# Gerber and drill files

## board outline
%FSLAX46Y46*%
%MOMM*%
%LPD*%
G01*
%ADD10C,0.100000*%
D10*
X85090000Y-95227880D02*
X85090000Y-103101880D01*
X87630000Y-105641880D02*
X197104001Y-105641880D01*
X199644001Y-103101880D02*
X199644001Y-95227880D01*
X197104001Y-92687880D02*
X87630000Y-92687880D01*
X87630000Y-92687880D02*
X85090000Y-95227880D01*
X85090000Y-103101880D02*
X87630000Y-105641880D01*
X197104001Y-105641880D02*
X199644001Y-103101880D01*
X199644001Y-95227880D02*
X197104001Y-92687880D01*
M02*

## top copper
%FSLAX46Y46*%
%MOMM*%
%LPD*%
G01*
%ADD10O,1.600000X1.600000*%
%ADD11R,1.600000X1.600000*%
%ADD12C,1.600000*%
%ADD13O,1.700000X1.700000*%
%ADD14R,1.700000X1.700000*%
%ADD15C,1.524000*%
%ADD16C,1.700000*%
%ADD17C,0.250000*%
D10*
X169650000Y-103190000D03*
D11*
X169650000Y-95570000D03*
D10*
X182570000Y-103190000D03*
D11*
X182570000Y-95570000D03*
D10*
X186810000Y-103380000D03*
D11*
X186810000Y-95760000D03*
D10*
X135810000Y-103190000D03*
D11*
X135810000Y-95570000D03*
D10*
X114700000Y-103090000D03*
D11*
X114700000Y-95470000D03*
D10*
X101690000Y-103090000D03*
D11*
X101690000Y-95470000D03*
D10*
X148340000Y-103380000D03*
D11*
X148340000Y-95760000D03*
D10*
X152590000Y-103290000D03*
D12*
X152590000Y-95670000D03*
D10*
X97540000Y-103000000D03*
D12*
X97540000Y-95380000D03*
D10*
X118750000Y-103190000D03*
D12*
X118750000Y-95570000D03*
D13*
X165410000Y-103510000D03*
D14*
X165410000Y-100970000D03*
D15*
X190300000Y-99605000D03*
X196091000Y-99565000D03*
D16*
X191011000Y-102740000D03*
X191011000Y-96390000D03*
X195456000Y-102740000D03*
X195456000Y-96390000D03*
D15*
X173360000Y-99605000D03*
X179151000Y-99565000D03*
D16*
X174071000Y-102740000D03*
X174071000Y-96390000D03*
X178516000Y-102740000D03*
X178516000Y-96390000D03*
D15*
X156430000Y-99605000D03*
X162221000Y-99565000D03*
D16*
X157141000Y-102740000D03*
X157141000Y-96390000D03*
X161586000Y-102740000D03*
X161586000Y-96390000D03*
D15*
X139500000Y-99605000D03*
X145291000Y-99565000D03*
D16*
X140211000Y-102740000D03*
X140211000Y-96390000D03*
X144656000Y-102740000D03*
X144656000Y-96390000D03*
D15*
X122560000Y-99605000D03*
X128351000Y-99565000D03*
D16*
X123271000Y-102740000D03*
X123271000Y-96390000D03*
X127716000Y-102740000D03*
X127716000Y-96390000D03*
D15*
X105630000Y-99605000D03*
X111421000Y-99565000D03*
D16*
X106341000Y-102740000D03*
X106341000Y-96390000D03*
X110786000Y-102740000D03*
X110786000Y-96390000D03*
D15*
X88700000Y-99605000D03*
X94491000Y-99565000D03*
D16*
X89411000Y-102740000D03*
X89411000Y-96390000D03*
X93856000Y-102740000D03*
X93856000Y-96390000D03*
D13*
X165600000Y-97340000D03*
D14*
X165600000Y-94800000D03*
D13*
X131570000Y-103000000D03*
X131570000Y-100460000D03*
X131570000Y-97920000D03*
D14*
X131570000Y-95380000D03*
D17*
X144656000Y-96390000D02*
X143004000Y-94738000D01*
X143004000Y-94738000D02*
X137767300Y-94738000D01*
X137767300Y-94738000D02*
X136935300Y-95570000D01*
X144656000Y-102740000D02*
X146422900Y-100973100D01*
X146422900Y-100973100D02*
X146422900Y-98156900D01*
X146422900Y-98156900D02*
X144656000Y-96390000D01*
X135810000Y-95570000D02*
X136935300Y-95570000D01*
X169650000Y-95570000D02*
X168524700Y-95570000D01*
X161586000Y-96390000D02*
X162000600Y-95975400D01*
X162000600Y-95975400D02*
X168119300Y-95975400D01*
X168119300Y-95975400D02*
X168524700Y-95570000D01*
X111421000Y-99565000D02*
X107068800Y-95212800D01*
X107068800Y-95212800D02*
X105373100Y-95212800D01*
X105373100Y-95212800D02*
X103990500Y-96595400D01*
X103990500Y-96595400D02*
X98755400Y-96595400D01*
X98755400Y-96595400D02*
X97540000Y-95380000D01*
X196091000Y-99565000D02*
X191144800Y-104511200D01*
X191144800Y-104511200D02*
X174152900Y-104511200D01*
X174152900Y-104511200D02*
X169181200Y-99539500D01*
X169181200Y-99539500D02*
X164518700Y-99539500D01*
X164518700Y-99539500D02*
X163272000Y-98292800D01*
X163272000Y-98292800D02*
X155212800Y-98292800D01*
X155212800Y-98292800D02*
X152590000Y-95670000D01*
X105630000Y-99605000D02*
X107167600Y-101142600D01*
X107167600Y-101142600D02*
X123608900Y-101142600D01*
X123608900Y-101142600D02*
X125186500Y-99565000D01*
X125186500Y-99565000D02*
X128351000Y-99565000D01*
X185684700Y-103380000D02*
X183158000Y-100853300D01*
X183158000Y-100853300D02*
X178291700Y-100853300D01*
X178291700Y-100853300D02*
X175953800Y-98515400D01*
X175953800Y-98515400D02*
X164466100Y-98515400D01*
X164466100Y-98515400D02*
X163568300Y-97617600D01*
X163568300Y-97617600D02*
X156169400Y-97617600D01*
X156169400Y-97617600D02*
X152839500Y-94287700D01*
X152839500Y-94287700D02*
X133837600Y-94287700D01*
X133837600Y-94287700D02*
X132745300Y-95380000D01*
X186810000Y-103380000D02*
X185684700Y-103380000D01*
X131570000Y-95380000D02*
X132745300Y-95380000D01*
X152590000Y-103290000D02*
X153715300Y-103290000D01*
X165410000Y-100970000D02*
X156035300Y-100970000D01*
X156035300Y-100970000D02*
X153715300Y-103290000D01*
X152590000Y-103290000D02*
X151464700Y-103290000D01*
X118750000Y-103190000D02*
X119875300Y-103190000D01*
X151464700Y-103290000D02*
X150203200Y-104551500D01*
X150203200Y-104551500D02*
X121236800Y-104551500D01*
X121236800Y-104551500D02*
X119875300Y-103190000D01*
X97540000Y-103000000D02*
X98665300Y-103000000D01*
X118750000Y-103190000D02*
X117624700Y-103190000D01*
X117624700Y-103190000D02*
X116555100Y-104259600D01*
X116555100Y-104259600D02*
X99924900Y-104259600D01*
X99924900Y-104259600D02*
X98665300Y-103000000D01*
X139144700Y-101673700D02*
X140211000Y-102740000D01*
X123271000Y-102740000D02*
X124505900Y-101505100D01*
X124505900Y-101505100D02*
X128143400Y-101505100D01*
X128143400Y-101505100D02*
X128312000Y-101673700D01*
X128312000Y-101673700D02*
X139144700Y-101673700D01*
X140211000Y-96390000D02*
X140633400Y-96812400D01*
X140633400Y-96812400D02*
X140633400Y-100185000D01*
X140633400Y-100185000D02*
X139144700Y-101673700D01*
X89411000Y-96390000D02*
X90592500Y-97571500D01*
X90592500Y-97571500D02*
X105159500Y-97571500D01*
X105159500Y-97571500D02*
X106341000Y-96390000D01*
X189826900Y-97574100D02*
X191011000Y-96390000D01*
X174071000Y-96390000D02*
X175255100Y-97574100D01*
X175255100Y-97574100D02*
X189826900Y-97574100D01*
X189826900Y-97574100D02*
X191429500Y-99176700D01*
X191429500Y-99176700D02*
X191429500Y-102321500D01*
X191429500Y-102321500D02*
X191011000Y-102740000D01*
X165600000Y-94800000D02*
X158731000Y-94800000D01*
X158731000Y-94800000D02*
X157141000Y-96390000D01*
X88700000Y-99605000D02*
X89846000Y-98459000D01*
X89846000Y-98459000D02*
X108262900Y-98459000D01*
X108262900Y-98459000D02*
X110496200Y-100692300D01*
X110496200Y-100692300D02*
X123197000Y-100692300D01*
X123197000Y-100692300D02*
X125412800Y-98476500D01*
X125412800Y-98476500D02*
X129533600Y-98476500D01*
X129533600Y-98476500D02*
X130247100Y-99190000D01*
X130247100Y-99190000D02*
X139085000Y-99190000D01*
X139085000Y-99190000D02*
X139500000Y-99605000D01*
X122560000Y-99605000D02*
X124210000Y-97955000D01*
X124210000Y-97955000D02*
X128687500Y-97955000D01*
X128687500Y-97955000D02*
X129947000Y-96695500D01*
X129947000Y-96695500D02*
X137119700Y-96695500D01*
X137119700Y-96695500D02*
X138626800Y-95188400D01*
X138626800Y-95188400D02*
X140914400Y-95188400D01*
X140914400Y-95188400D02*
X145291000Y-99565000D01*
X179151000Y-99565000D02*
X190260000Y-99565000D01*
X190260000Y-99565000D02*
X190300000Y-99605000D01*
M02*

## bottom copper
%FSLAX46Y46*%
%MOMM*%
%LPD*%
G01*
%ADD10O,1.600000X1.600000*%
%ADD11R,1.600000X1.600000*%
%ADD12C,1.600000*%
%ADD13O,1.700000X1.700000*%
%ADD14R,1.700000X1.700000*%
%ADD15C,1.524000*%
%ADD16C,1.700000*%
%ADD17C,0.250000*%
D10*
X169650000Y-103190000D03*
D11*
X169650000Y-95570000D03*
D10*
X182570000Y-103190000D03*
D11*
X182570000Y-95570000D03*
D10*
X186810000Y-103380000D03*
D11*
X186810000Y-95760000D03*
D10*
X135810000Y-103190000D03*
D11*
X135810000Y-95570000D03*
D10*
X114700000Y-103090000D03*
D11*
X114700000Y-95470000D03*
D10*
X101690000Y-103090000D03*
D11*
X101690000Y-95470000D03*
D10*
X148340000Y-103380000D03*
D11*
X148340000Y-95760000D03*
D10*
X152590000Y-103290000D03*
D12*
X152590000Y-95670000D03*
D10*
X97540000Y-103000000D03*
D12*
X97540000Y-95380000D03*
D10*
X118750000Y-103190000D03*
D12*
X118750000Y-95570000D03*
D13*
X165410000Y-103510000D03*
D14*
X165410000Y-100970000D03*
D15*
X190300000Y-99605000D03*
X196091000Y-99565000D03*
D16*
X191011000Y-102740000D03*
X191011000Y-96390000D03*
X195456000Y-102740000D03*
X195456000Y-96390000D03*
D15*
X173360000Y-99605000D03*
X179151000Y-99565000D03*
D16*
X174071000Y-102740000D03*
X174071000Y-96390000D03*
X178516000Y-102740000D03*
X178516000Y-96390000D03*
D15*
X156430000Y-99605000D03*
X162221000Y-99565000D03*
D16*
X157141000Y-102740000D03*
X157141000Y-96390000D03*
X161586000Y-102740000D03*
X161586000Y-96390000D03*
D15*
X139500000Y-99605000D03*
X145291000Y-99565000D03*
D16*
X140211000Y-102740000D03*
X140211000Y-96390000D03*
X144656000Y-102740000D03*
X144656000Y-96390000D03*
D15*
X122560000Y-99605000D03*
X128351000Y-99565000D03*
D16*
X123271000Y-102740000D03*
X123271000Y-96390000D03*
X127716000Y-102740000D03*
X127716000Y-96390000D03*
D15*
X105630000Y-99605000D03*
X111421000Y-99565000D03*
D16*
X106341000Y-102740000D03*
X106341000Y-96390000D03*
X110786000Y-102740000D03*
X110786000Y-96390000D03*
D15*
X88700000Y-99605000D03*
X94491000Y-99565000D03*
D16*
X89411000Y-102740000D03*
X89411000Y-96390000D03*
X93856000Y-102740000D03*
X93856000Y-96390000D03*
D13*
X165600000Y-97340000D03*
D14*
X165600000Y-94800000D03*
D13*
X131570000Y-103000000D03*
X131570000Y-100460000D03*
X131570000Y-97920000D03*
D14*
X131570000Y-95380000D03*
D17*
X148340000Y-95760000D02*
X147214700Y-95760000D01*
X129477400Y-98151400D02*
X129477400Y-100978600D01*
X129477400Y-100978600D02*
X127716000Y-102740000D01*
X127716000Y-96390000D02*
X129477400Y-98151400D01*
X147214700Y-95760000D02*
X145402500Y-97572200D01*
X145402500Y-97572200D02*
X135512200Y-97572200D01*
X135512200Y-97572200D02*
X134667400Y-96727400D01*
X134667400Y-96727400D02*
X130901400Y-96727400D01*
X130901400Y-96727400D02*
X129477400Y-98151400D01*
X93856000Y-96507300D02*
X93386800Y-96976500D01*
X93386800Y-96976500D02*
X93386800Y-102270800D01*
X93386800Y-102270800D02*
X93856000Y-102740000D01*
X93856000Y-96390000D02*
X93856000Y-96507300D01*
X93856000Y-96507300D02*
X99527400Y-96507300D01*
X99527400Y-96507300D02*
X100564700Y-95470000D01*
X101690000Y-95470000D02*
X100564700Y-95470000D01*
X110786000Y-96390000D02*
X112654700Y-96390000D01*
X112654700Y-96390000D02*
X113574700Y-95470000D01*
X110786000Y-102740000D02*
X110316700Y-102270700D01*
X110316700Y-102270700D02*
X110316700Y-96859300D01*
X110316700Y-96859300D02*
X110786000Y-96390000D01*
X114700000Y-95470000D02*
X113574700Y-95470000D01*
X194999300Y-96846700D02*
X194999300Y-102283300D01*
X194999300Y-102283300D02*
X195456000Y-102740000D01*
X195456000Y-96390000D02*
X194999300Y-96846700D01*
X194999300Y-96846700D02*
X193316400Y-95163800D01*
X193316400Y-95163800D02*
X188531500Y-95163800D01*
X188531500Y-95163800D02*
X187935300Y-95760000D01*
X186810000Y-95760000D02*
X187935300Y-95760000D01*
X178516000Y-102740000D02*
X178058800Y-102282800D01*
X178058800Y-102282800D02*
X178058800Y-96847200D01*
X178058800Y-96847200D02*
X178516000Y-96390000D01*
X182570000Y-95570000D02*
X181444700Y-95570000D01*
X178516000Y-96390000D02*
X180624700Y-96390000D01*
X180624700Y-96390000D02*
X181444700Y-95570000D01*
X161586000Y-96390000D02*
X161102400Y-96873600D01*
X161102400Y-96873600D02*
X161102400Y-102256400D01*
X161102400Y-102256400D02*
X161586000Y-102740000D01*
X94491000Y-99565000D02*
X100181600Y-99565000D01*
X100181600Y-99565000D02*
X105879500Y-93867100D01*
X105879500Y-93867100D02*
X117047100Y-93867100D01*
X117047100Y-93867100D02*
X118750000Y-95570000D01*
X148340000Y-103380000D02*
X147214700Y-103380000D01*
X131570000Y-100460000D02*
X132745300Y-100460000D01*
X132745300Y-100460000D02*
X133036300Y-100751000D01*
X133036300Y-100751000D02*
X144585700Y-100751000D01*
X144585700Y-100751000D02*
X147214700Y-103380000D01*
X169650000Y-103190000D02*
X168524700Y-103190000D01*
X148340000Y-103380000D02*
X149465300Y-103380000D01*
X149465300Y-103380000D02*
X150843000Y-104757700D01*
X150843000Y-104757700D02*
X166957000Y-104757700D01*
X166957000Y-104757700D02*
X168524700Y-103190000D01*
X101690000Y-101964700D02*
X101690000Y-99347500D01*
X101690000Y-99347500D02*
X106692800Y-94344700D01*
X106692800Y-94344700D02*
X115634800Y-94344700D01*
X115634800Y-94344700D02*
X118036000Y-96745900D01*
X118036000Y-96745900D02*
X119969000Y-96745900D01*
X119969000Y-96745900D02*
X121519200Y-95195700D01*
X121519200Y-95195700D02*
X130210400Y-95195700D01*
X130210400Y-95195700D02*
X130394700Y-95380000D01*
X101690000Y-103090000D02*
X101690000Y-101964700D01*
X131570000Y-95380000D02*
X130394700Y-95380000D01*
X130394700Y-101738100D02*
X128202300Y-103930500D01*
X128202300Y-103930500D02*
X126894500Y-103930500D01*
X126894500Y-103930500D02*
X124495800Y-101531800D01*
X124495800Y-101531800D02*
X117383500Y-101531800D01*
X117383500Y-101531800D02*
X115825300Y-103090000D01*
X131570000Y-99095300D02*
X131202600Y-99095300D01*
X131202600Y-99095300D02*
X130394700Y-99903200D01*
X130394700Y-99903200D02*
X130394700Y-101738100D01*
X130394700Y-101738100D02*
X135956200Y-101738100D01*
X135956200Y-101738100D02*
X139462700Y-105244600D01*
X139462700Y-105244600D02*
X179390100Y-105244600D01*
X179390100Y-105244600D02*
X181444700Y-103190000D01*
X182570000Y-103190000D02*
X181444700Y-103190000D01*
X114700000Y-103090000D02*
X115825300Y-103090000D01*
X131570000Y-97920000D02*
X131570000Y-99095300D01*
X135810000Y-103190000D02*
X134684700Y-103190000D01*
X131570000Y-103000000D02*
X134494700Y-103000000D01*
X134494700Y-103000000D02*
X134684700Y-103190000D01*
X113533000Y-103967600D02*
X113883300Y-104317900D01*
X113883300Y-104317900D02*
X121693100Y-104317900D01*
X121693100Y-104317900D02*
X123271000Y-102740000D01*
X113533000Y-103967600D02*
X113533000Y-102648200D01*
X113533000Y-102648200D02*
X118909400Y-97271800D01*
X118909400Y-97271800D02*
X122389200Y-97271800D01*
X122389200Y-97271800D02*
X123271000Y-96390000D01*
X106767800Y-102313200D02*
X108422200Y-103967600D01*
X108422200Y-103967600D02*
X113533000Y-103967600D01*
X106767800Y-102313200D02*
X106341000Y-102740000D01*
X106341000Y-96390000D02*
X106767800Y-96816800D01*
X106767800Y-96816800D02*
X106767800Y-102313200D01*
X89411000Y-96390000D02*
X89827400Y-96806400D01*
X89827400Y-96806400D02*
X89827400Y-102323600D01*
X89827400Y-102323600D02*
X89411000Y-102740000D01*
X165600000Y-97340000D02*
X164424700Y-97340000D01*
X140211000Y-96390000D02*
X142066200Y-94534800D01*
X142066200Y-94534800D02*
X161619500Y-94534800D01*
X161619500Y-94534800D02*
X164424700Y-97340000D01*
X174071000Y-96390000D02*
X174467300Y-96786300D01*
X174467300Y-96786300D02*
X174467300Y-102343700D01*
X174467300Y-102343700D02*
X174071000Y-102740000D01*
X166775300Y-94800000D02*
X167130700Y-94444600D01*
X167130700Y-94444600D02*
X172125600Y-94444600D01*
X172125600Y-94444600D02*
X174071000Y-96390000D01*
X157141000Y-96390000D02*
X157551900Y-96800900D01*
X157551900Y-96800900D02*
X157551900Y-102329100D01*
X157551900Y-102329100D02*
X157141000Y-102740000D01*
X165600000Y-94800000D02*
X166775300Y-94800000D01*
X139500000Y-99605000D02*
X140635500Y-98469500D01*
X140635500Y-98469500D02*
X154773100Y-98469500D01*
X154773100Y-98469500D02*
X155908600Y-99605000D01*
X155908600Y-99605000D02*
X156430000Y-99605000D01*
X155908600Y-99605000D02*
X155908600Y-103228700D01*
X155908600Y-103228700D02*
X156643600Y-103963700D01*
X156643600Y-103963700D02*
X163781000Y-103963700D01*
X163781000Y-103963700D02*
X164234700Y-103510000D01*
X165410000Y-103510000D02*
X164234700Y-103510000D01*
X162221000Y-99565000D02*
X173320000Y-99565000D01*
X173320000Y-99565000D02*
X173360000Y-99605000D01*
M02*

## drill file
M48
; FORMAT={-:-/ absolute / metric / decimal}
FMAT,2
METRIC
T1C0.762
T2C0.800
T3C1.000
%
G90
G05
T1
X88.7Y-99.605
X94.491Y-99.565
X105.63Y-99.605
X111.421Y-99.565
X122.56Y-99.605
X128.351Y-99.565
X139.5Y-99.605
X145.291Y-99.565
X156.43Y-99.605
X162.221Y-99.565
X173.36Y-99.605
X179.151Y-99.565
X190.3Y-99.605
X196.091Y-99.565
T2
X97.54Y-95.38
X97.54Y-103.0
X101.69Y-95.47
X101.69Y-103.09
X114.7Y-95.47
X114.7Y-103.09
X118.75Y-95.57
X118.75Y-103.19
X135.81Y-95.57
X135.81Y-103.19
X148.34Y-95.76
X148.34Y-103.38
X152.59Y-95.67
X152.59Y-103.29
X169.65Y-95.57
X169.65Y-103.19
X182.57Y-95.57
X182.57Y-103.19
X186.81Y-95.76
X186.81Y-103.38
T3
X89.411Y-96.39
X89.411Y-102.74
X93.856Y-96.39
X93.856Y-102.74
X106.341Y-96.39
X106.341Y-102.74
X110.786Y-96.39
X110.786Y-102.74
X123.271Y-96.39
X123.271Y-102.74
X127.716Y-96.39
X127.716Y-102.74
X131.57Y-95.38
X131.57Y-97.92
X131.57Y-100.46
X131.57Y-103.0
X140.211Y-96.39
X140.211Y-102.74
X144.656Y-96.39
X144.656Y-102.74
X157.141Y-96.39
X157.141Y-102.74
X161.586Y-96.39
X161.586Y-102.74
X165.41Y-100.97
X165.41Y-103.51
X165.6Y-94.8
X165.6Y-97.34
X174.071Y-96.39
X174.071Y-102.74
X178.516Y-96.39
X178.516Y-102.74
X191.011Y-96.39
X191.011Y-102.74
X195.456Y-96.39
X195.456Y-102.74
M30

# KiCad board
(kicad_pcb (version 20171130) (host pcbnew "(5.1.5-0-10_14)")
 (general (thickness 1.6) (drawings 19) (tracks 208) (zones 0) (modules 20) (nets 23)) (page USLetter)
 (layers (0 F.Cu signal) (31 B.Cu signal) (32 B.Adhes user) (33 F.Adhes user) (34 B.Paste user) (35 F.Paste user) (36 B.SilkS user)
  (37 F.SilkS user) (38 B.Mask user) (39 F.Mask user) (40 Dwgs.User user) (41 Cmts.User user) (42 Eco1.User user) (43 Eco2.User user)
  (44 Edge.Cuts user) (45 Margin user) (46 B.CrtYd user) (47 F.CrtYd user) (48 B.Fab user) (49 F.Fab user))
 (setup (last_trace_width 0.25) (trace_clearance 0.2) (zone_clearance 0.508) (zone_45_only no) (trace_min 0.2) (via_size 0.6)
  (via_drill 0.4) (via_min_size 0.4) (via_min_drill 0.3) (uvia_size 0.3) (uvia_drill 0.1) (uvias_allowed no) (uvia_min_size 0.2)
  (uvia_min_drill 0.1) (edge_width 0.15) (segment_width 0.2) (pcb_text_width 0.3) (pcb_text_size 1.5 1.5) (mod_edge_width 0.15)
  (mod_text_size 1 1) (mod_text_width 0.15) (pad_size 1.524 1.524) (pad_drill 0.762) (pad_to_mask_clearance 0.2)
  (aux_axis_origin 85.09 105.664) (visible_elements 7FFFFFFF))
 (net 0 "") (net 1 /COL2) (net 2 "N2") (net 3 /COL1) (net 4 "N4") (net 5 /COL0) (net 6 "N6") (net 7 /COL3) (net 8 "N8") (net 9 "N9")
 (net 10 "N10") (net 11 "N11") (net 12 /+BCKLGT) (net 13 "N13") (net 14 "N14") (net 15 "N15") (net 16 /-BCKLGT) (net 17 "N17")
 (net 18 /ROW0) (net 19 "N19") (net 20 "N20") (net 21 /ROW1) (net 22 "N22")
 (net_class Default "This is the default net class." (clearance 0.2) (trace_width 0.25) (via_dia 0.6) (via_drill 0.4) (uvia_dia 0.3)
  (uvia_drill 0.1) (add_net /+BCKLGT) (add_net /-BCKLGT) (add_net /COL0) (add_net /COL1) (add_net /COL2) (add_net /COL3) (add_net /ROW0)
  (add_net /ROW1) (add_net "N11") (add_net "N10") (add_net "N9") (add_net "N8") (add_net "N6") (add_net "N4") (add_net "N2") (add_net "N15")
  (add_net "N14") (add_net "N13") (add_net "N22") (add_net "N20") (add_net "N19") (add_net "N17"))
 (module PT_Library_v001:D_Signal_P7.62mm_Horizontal (layer F.Cu) (at 169.65 95.57 270)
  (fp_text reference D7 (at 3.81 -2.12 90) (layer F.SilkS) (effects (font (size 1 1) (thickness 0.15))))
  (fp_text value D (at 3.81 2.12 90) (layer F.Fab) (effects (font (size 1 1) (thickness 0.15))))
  (pad 2 thru_hole oval (at 7.62 0 270) (size 1.6 1.6) (drill 0.8) (layers *.Cu *.Mask) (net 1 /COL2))
  (pad 1 thru_hole rect (at 0 0 270) (size 1.6 1.6) (drill 0.8) (layers *.Cu *.Mask) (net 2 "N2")))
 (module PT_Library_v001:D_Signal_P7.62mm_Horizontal (layer F.Cu) (at 182.57 95.57 270)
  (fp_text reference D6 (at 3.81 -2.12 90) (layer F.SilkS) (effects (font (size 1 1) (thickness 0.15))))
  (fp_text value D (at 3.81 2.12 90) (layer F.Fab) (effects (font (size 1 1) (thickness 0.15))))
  (pad 2 thru_hole oval (at 7.62 0 270) (size 1.6 1.6) (drill 0.8) (layers *.Cu *.Mask) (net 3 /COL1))
  (pad 1 thru_hole rect (at 0 0 270) (size 1.6 1.6) (drill 0.8) (layers *.Cu *.Mask) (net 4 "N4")))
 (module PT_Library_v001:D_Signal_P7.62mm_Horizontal (layer F.Cu) (at 186.81 95.76 270)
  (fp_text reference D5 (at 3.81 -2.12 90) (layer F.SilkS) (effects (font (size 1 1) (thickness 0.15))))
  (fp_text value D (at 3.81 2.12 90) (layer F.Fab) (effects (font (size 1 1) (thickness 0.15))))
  (pad 2 thru_hole oval (at 7.62 0 270) (size 1.6 1.6) (drill 0.8) (layers *.Cu *.Mask) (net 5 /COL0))
  (pad 1 thru_hole rect (at 0 0 270) (size 1.6 1.6) (drill 0.8) (layers *.Cu *.Mask) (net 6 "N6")))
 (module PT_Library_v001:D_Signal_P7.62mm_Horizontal (layer F.Cu) (at 135.81 95.57 270)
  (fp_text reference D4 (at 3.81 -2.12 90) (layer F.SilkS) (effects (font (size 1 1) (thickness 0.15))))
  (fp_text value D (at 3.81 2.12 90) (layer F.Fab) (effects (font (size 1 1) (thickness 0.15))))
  (pad 2 thru_hole oval (at 7.62 0 270) (size 1.6 1.6) (drill 0.8) (layers *.Cu *.Mask) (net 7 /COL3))
  (pad 1 thru_hole rect (at 0 0 270) (size 1.6 1.6) (drill 0.8) (layers *.Cu *.Mask) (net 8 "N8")))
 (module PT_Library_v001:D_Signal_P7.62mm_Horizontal (layer F.Cu) (at 114.7 95.47 270)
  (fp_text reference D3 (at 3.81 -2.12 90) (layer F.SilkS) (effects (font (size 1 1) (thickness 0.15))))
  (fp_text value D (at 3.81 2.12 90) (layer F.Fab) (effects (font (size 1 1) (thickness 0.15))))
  (pad 2 thru_hole oval (at 7.62 0 270) (size 1.6 1.6) (drill 0.8) (layers *.Cu *.Mask) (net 3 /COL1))
  (pad 1 thru_hole rect (at 0 0 270) (size 1.6 1.6) (drill 0.8) (layers *.Cu *.Mask) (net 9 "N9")))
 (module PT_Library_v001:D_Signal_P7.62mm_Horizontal (layer F.Cu) (at 101.69 95.47 270)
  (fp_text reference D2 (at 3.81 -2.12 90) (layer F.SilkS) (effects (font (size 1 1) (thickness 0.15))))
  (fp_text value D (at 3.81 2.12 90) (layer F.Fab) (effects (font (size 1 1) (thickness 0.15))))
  (pad 2 thru_hole oval (at 7.62 0 270) (size 1.6 1.6) (drill 0.8) (layers *.Cu *.Mask) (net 5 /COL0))
  (pad 1 thru_hole rect (at 0 0 270) (size 1.6 1.6) (drill 0.8) (layers *.Cu *.Mask) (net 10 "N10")))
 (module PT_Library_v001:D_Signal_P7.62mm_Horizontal (layer F.Cu) (at 148.34 95.76 270)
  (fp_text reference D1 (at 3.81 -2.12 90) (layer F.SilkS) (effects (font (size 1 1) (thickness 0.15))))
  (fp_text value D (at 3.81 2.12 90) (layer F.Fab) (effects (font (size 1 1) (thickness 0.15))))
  (pad 2 thru_hole oval (at 7.62 0 270) (size 1.6 1.6) (drill 0.8) (layers *.Cu *.Mask) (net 1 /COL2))
  (pad 1 thru_hole rect (at 0 0 270) (size 1.6 1.6) (drill 0.8) (layers *.Cu *.Mask) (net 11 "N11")))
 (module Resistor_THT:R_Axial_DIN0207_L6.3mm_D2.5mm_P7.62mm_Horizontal (layer F.Cu) (at 152.59 95.67 270)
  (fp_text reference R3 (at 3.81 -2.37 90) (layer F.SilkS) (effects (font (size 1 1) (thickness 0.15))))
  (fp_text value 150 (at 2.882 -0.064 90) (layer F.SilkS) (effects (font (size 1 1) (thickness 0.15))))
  (pad 2 thru_hole oval (at 7.62 0 270) (size 1.6 1.6) (drill 0.8) (layers *.Cu *.Mask) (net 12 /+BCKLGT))
  (pad 1 thru_hole circle (at 0 0 270) (size 1.6 1.6) (drill 0.8) (layers *.Cu *.Mask) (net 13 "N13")))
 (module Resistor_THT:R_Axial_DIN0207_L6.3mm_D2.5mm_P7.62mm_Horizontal (layer F.Cu) (at 97.54 95.38 270)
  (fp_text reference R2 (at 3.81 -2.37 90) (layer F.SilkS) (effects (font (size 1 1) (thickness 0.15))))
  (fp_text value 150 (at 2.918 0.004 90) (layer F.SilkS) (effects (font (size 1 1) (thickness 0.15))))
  (pad 2 thru_hole oval (at 7.62 0 270) (size 1.6 1.6) (drill 0.8) (layers *.Cu *.Mask) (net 12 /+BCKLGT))
  (pad 1 thru_hole circle (at 0 0 270) (size 1.6 1.6) (drill 0.8) (layers *.Cu *.Mask) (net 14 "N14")))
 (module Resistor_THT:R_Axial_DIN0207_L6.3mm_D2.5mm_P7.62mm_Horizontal (layer F.Cu) (at 118.75 95.57 270)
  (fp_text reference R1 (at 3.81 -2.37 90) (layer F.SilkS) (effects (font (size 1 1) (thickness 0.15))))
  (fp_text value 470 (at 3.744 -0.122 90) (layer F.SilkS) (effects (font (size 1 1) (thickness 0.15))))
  (pad 2 thru_hole oval (at 7.62 0 270) (size 1.6 1.6) (drill 0.8) (layers *.Cu *.Mask) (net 12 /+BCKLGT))
  (pad 1 thru_hole circle (at 0 0 270) (size 1.6 1.6) (drill 0.8) (layers *.Cu *.Mask) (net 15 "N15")))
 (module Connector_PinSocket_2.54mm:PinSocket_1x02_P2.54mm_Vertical (layer B.Cu) (at 165.41 100.97 180)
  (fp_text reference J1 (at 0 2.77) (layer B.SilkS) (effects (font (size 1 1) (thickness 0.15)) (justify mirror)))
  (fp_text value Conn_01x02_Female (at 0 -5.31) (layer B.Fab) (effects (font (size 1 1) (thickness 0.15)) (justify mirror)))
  (pad 2 thru_hole oval (at 0 -2.54 180) (size 1.7 1.7) (drill 1) (layers *.Cu *.Mask) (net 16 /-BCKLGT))
  (pad 1 thru_hole rect (at 0 0 180) (size 1.7 1.7) (drill 1) (layers *.Cu *.Mask) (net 12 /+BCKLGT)))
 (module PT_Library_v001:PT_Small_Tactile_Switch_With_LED (layer F.Cu) (at 193.17 99.565 270)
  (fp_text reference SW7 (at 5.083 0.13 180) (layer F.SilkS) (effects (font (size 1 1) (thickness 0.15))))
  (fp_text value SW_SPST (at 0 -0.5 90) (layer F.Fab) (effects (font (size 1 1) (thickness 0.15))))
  (pad 6 thru_hole circle (at 0.04 2.87 270) (size 1.524 1.524) (drill 0.762) (layers *.Cu *.Mask) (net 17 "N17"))
  (pad 5 thru_hole circle (at 0 -2.921 270) (size 1.524 1.524) (drill 0.762) (layers *.Cu *.Mask) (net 13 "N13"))
  (pad 4 thru_hole circle (at 3.175 2.159 270) (size 1.7 1.7) (drill 1) (layers *.Cu *.Mask) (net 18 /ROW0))
  (pad 3 thru_hole circle (at -3.175 2.159 270) (size 1.7 1.7) (drill 1) (layers *.Cu *.Mask) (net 18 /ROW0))
  (pad 2 thru_hole circle (at 3.175 -2.286 270) (size 1.7 1.7) (drill 1) (layers *.Cu *.Mask) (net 6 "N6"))
  (pad 1 thru_hole circle (at -3.175 -2.286 270) (size 1.7 1.7) (drill 1) (layers *.Cu *.Mask) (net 6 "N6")))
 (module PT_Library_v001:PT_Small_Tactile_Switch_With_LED (layer F.Cu) (at 176.23 99.565 270)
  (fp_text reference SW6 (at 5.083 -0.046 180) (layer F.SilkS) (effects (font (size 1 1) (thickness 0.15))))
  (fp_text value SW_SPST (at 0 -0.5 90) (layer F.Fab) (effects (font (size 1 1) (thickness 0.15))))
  (pad 6 thru_hole circle (at 0.04 2.87 270) (size 1.524 1.524) (drill 0.762) (layers *.Cu *.Mask) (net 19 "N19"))
  (pad 5 thru_hole circle (at 0 -2.921 270) (size 1.524 1.524) (drill 0.762) (layers *.Cu *.Mask) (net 17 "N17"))
  (pad 4 thru_hole circle (at 3.175 2.159 270) (size 1.7 1.7) (drill 1) (layers *.Cu *.Mask) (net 18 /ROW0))
  (pad 3 thru_hole circle (at -3.175 2.159 270) (size 1.7 1.7) (drill 1) (layers *.Cu *.Mask) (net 18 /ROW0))
  (pad 2 thru_hole circle (at 3.175 -2.286 270) (size 1.7 1.7) (drill 1) (layers *.Cu *.Mask) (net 4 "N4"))
  (pad 1 thru_hole circle (at -3.175 -2.286 270) (size 1.7 1.7) (drill 1) (layers *.Cu *.Mask) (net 4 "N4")))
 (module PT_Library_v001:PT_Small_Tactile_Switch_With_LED (layer F.Cu) (at 159.3 99.565 270)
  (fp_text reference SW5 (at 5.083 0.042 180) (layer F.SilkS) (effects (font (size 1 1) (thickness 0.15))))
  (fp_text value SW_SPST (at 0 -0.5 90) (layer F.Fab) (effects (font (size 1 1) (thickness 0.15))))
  (pad 6 thru_hole circle (at 0.04 2.87 270) (size 1.524 1.524) (drill 0.762) (layers *.Cu *.Mask) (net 16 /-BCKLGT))
  (pad 5 thru_hole circle (at 0 -2.921 270) (size 1.524 1.524) (drill 0.762) (layers *.Cu *.Mask) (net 19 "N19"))
  (pad 4 thru_hole circle (at 3.175 2.159 270) (size 1.7 1.7) (drill 1) (layers *.Cu *.Mask) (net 18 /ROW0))
  (pad 3 thru_hole circle (at -3.175 2.159 270) (size 1.7 1.7) (drill 1) (layers *.Cu *.Mask) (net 18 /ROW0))
  (pad 2 thru_hole circle (at 3.175 -2.286 270) (size 1.7 1.7) (drill 1) (layers *.Cu *.Mask) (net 2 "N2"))
  (pad 1 thru_hole circle (at -3.175 -2.286 270) (size 1.7 1.7) (drill 1) (layers *.Cu *.Mask) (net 2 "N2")))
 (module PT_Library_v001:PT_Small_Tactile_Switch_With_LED (layer F.Cu) (at 142.37 99.565 270)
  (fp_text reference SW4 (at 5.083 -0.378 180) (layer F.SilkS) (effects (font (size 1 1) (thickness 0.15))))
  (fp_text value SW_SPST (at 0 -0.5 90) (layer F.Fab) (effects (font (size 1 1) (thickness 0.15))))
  (pad 6 thru_hole circle (at 0.04 2.87 270) (size 1.524 1.524) (drill 0.762) (layers *.Cu *.Mask) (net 16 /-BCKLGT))
  (pad 5 thru_hole circle (at 0 -2.921 270) (size 1.524 1.524) (drill 0.762) (layers *.Cu *.Mask) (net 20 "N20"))
  (pad 4 thru_hole circle (at 3.175 2.159 270) (size 1.7 1.7) (drill 1) (layers *.Cu *.Mask) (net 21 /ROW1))
  (pad 3 thru_hole circle (at -3.175 2.159 270) (size 1.7 1.7) (drill 1) (layers *.Cu *.Mask) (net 21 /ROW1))
  (pad 2 thru_hole circle (at 3.175 -2.286 270) (size 1.7 1.7) (drill 1) (layers *.Cu *.Mask) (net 8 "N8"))
  (pad 1 thru_hole circle (at -3.175 -2.286 270) (size 1.7 1.7) (drill 1) (layers *.Cu *.Mask) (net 8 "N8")))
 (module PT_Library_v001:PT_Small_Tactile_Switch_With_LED (layer F.Cu) (at 125.43 99.565 270)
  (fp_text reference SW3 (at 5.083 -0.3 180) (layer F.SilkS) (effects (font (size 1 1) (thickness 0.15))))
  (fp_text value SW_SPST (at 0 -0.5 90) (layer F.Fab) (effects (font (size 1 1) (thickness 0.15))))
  (pad 6 thru_hole circle (at 0.04 2.87 270) (size 1.524 1.524) (drill 0.762) (layers *.Cu *.Mask) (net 20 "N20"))
  (pad 5 thru_hole circle (at 0 -2.921 270) (size 1.524 1.524) (drill 0.762) (layers *.Cu *.Mask) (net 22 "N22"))
  (pad 4 thru_hole circle (at 3.175 2.159 270) (size 1.7 1.7) (drill 1) (layers *.Cu *.Mask) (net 21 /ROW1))
  (pad 3 thru_hole circle (at -3.175 2.159 270) (size 1.7 1.7) (drill 1) (layers *.Cu *.Mask) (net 21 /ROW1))
  (pad 2 thru_hole circle (at 3.175 -2.286 270) (size 1.7 1.7) (drill 1) (layers *.Cu *.Mask) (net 11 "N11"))
  (pad 1 thru_hole circle (at -3.175 -2.286 270) (size 1.7 1.7) (drill 1) (layers *.Cu *.Mask) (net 11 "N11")))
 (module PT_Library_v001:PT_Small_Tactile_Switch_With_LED (layer F.Cu) (at 108.5 99.565 270)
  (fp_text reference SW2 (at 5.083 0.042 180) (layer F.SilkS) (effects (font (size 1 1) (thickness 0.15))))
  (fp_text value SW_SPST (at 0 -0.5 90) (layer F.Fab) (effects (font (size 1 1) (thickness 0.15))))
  (pad 6 thru_hole circle (at 0.04 2.87 270) (size 1.524 1.524) (drill 0.762) (layers *.Cu *.Mask) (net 22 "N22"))
  (pad 5 thru_hole circle (at 0 -2.921 270) (size 1.524 1.524) (drill 0.762) (layers *.Cu *.Mask) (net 14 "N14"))
  (pad 4 thru_hole circle (at 3.175 2.159 270) (size 1.7 1.7) (drill 1) (layers *.Cu *.Mask) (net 21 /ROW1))
  (pad 3 thru_hole circle (at -3.175 2.159 270) (size 1.7 1.7) (drill 1) (layers *.Cu *.Mask) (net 21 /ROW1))
  (pad 2 thru_hole circle (at 3.175 -2.286 270) (size 1.7 1.7) (drill 1) (layers *.Cu *.Mask) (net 9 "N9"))
  (pad 1 thru_hole circle (at -3.175 -2.286 270) (size 1.7 1.7) (drill 1) (layers *.Cu *.Mask) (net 9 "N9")))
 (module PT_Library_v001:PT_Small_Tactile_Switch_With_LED (layer F.Cu) (at 91.57 99.565 270)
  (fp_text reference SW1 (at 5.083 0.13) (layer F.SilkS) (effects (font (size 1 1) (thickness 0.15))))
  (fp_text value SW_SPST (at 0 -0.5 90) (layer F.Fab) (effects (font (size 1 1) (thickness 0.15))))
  (pad 6 thru_hole circle (at 0.04 2.87 270) (size 1.524 1.524) (drill 0.762) (layers *.Cu *.Mask) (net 16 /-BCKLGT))
  (pad 5 thru_hole circle (at 0 -2.921 270) (size 1.524 1.524) (drill 0.762) (layers *.Cu *.Mask) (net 15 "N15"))
  (pad 4 thru_hole circle (at 3.175 2.159 270) (size 1.7 1.7) (drill 1) (layers *.Cu *.Mask) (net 21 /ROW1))
  (pad 3 thru_hole circle (at -3.175 2.159 270) (size 1.7 1.7) (drill 1) (layers *.Cu *.Mask) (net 21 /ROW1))
  (pad 2 thru_hole circle (at 3.175 -2.286 270) (size 1.7 1.7) (drill 1) (layers *.Cu *.Mask) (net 10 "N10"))
  (pad 1 thru_hole circle (at -3.175 -2.286 270) (size 1.7 1.7) (drill 1) (layers *.Cu *.Mask) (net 10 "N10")))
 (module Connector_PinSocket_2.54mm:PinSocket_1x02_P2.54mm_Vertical (layer B.Cu) (at 165.6 94.8 180)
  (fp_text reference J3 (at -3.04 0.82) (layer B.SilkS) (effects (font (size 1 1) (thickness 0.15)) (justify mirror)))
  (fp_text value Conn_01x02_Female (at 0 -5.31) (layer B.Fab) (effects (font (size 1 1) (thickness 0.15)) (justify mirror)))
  (pad 2 thru_hole oval (at 0 -2.54 180) (size 1.7 1.7) (drill 1) (layers *.Cu *.Mask) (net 21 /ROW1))
  (pad 1 thru_hole rect (at 0 0 180) (size 1.7 1.7) (drill 1) (layers *.Cu *.Mask) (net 18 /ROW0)))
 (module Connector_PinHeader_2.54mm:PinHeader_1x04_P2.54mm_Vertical (layer B.Cu) (at 131.57 95.38 180)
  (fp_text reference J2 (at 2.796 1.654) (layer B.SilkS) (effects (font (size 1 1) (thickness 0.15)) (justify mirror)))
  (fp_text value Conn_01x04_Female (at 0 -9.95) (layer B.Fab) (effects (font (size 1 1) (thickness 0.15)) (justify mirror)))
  (pad 4 thru_hole oval (at 0 -7.62 180) (size 1.7 1.7) (drill 1) (layers *.Cu *.Mask) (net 7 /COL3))
  (pad 3 thru_hole oval (at 0 -5.08 180) (size 1.7 1.7) (drill 1) (layers *.Cu *.Mask) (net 1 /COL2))
  (pad 2 thru_hole oval (at 0 -2.54 180) (size 1.7 1.7) (drill 1) (layers *.Cu *.Mask) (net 3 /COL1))
  (pad 1 thru_hole rect (at 0 0 180) (size 1.7 1.7) (drill 1) (layers *.Cu *.Mask) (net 5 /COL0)))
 (gr_line (start 85.09 95.22788) (end 85.09 103.10188) (layer Edge.Cuts) (width 0.1))
 (gr_line (start 87.63 105.64188) (end 197.104001 105.64188) (layer Edge.Cuts) (width 0.1))
 (gr_line (start 199.644001 103.10188) (end 199.644001 95.22788) (layer Edge.Cuts) (width 0.1))
 (gr_line (start 197.104001 92.68788) (end 87.63 92.68788) (layer Edge.Cuts) (width 0.1))
 (gr_line (start 87.63 92.68788) (end 85.09 95.22788) (layer Edge.Cuts) (width 0.1))
 (gr_line (start 85.09 103.10188) (end 87.63 105.64188) (layer Edge.Cuts) (width 0.1))
 (gr_line (start 197.104001 105.64188) (end 199.644001 103.10188) (layer Edge.Cuts) (width 0.1))
 (gr_line (start 199.644001 95.22788) (end 197.104001 92.68788) (layer Edge.Cuts) (width 0.1))
 (segment (start 148.34 95.76) (end 147.2147 95.76) (width 0.25) (layer B.Cu) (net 11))
 (segment (start 129.4774 98.1514) (end 129.4774 100.9786) (width 0.25) (layer B.Cu) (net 11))
 (segment (start 129.4774 100.9786) (end 127.716 102.74) (width 0.25) (layer B.Cu) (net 11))
 (segment (start 127.716 96.39) (end 129.4774 98.1514) (width 0.25) (layer B.Cu) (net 11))
 (segment (start 147.2147 95.76) (end 145.4025 97.5722) (width 0.25) (layer B.Cu) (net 11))
 (segment (start 145.4025 97.5722) (end 135.5122 97.5722) (width 0.25) (layer B.Cu) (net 11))
 (segment (start 135.5122 97.5722) (end 134.6674 96.7274) (width 0.25) (layer B.Cu) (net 11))
 (segment (start 134.6674 96.7274) (end 130.9014 96.7274) (width 0.25) (layer B.Cu) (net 11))
 (segment (start 130.9014 96.7274) (end 129.4774 98.1514) (width 0.25) (layer B.Cu) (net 11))
 (segment (start 93.856 96.5073) (end 93.3868 96.9765) (width 0.25) (layer B.Cu) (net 10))
 (segment (start 93.3868 96.9765) (end 93.3868 102.2708) (width 0.25) (layer B.Cu) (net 10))
 (segment (start 93.3868 102.2708) (end 93.856 102.74) (width 0.25) (layer B.Cu) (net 10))
 (segment (start 93.856 96.39) (end 93.856 96.5073) (width 0.25) (layer B.Cu) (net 10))
 (segment (start 93.856 96.5073) (end 99.5274 96.5073) (width 0.25) (layer B.Cu) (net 10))
 (segment (start 99.5274 96.5073) (end 100.5647 95.47) (width 0.25) (layer B.Cu) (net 10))
 (segment (start 101.69 95.47) (end 100.5647 95.47) (width 0.25) (layer B.Cu) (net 10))
 (segment (start 110.786 96.39) (end 112.6547 96.39) (width 0.25) (layer B.Cu) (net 9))
 (segment (start 112.6547 96.39) (end 113.5747 95.47) (width 0.25) (layer B.Cu) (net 9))
 (segment (start 110.786 102.74) (end 110.3167 102.2707) (width 0.25) (layer B.Cu) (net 9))
 (segment (start 110.3167 102.2707) (end 110.3167 96.8593) (width 0.25) (layer B.Cu) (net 9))
 (segment (start 110.3167 96.8593) (end 110.786 96.39) (width 0.25) (layer B.Cu) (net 9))
 (segment (start 114.7 95.47) (end 113.5747 95.47) (width 0.25) (layer B.Cu) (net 9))
 (segment (start 144.656 96.39) (end 143.004 94.738) (width 0.25) (layer F.Cu) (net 8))
 (segment (start 143.004 94.738) (end 137.7673 94.738) (width 0.25) (layer F.Cu) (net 8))
 (segment (start 137.7673 94.738) (end 136.9353 95.57) (width 0.25) (layer F.Cu) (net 8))
 (segment (start 144.656 102.74) (end 146.4229 100.9731) (width 0.25) (layer F.Cu) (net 8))
 (segment (start 146.4229 100.9731) (end 146.4229 98.1569) (width 0.25) (layer F.Cu) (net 8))
 (segment (start 146.4229 98.1569) (end 144.656 96.39) (width 0.25) (layer F.Cu) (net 8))
 (segment (start 135.81 95.57) (end 136.9353 95.57) (width 0.25) (layer F.Cu) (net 8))
 (segment (start 194.9993 96.8467) (end 194.9993 102.2833) (width 0.25) (layer B.Cu) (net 6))
 (segment (start 194.9993 102.2833) (end 195.456 102.74) (width 0.25) (layer B.Cu) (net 6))
 (segment (start 195.456 96.39) (end 194.9993 96.8467) (width 0.25) (layer B.Cu) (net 6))
 (segment (start 194.9993 96.8467) (end 193.3164 95.1638) (width 0.25) (layer B.Cu) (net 6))
 (segment (start 193.3164 95.1638) (end 188.5315 95.1638) (width 0.25) (layer B.Cu) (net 6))
 (segment (start 188.5315 95.1638) (end 187.9353 95.76) (width 0.25) (layer B.Cu) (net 6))
 (segment (start 186.81 95.76) (end 187.9353 95.76) (width 0.25) (layer B.Cu) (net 6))
 (segment (start 178.516 102.74) (end 178.0588 102.2828) (width 0.25) (layer B.Cu) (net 4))
 (segment (start 178.0588 102.2828) (end 178.0588 96.8472) (width 0.25) (layer B.Cu) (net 4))
 (segment (start 178.0588 96.8472) (end 178.516 96.39) (width 0.25) (layer B.Cu) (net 4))
 (segment (start 182.57 95.57) (end 181.4447 95.57) (width 0.25) (layer B.Cu) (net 4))
 (segment (start 178.516 96.39) (end 180.6247 96.39) (width 0.25) (layer B.Cu) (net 4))
 (segment (start 180.6247 96.39) (end 181.4447 95.57) (width 0.25) (layer B.Cu) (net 4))
 (segment (start 169.65 95.57) (end 168.5247 95.57) (width 0.25) (layer F.Cu) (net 2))
 (segment (start 161.586 96.39) (end 162.0006 95.9754) (width 0.25) (layer F.Cu) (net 2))
 (segment (start 162.0006 95.9754) (end 168.1193 95.9754) (width 0.25) (layer F.Cu) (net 2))
 (segment (start 168.1193 95.9754) (end 168.5247 95.57) (width 0.25) (layer F.Cu) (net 2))
 (segment (start 161.586 96.39) (end 161.1024 96.8736) (width 0.25) (layer B.Cu) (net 2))
 (segment (start 161.1024 96.8736) (end 161.1024 102.2564) (width 0.25) (layer B.Cu) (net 2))
 (segment (start 161.1024 102.2564) (end 161.586 102.74) (width 0.25) (layer B.Cu) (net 2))
 (segment (start 94.491 99.565) (end 100.1816 99.565) (width 0.25) (layer B.Cu) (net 15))
 (segment (start 100.1816 99.565) (end 105.8795 93.8671) (width 0.25) (layer B.Cu) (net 15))
 (segment (start 105.8795 93.8671) (end 117.0471 93.8671) (width 0.25) (layer B.Cu) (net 15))
 (segment (start 117.0471 93.8671) (end 118.75 95.57) (width 0.25) (layer B.Cu) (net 15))
 (segment (start 111.421 99.565) (end 107.0688 95.2128) (width 0.25) (layer F.Cu) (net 14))
 (segment (start 107.0688 95.2128) (end 105.3731 95.2128) (width 0.25) (layer F.Cu) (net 14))
 (segment (start 105.3731 95.2128) (end 103.9905 96.5954) (width 0.25) (layer F.Cu) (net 14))
 (segment (start 103.9905 96.5954) (end 98.7554 96.5954) (width 0.25) (layer F.Cu) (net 14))
 (segment (start 98.7554 96.5954) (end 97.54 95.38) (width 0.25) (layer F.Cu) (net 14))
 (segment (start 196.091 99.565) (end 191.1448 104.5112) (width 0.25) (layer F.Cu) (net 13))
 (segment (start 191.1448 104.5112) (end 174.1529 104.5112) (width 0.25) (layer F.Cu) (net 13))
 (segment (start 174.1529 104.5112) (end 169.1812 99.5395) (width 0.25) (layer F.Cu) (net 13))
 (segment (start 169.1812 99.5395) (end 164.5187 99.5395) (width 0.25) (layer F.Cu) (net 13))
 (segment (start 164.5187 99.5395) (end 163.272 98.2928) (width 0.25) (layer F.Cu) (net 13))
 (segment (start 163.272 98.2928) (end 155.2128 98.2928) (width 0.25) (layer F.Cu) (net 13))
 (segment (start 155.2128 98.2928) (end 152.59 95.67) (width 0.25) (layer F.Cu) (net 13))
 (segment (start 105.63 99.605) (end 107.1676 101.1426) (width 0.25) (layer F.Cu) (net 22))
 (segment (start 107.1676 101.1426) (end 123.6089 101.1426) (width 0.25) (layer F.Cu) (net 22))
 (segment (start 123.6089 101.1426) (end 125.1865 99.565) (width 0.25) (layer F.Cu) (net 22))
 (segment (start 125.1865 99.565) (end 128.351 99.565) (width 0.25) (layer F.Cu) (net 22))
 (segment (start 148.34 103.38) (end 147.2147 103.38) (width 0.25) (layer B.Cu) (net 1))
 (segment (start 131.57 100.46) (end 132.7453 100.46) (width 0.25) (layer B.Cu) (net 1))
 (segment (start 132.7453 100.46) (end 133.0363 100.751) (width 0.25) (layer B.Cu) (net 1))
 (segment (start 133.0363 100.751) (end 144.5857 100.751) (width 0.25) (layer B.Cu) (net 1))
 (segment (start 144.5857 100.751) (end 147.2147 103.38) (width 0.25) (layer B.Cu) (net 1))
 (segment (start 169.65 103.19) (end 168.5247 103.19) (width 0.25) (layer B.Cu) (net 1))
 (segment (start 148.34 103.38) (end 149.4653 103.38) (width 0.25) (layer B.Cu) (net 1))
 (segment (start 149.4653 103.38) (end 150.843 104.7577) (width 0.25) (layer B.Cu) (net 1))
 (segment (start 150.843 104.7577) (end 166.957 104.7577) (width 0.25) (layer B.Cu) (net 1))
 (segment (start 166.957 104.7577) (end 168.5247 103.19) (width 0.25) (layer B.Cu) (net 1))
 (segment (start 185.6847 103.38) (end 183.158 100.8533) (width 0.25) (layer F.Cu) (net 5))
 (segment (start 183.158 100.8533) (end 178.2917 100.8533) (width 0.25) (layer F.Cu) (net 5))
 (segment (start 178.2917 100.8533) (end 175.9538 98.5154) (width 0.25) (layer F.Cu) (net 5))
 (segment (start 175.9538 98.5154) (end 164.4661 98.5154) (width 0.25) (layer F.Cu) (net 5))
 (segment (start 164.4661 98.5154) (end 163.5683 97.6176) (width 0.25) (layer F.Cu) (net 5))
 (segment (start 163.5683 97.6176) (end 156.1694 97.6176) (width 0.25) (layer F.Cu) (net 5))
 (segment (start 156.1694 97.6176) (end 152.8395 94.2877) (width 0.25) (layer F.Cu) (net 5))
 (segment (start 152.8395 94.2877) (end 133.8376 94.2877) (width 0.25) (layer F.Cu) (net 5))
 (segment (start 133.8376 94.2877) (end 132.7453 95.38) (width 0.25) (layer F.Cu) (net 5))
 (segment (start 101.69 101.9647) (end 101.69 99.3475) (width 0.25) (layer B.Cu) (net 5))
 (segment (start 101.69 99.3475) (end 106.6928 94.3447) (width 0.25) (layer B.Cu) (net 5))
 (segment (start 106.6928 94.3447) (end 115.6348 94.3447) (width 0.25) (layer B.Cu) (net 5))
 (segment (start 115.6348 94.3447) (end 118.036 96.7459) (width 0.25) (layer B.Cu) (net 5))
 (segment (start 118.036 96.7459) (end 119.969 96.7459) (width 0.25) (layer B.Cu) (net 5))
 (segment (start 119.969 96.7459) (end 121.5192 95.1957) (width 0.25) (layer B.Cu) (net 5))
 (segment (start 121.5192 95.1957) (end 130.2104 95.1957) (width 0.25) (layer B.Cu) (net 5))
 (segment (start 130.2104 95.1957) (end 130.3947 95.38) (width 0.25) (layer B.Cu) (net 5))
 (segment (start 186.81 103.38) (end 185.6847 103.38) (width 0.25) (layer F.Cu) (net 5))
 (segment (start 131.57 95.38) (end 132.7453 95.38) (width 0.25) (layer F.Cu) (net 5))
 (segment (start 101.69 103.09) (end 101.69 101.9647) (width 0.25) (layer B.Cu) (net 5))
 (segment (start 131.57 95.38) (end 130.3947 95.38) (width 0.25) (layer B.Cu) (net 5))
 (segment (start 130.3947 101.7381) (end 128.2023 103.9305) (width 0.25) (layer B.Cu) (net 3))
 (segment (start 128.2023 103.9305) (end 126.8945 103.9305) (width 0.25) (layer B.Cu) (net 3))
 (segment (start 126.8945 103.9305) (end 124.4958 101.5318) (width 0.25) (layer B.Cu) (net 3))
 (segment (start 124.4958 101.5318) (end 117.3835 101.5318) (width 0.25) (layer B.Cu) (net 3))
 (segment (start 117.3835 101.5318) (end 115.8253 103.09) (width 0.25) (layer B.Cu) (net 3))
 (segment (start 131.57 99.0953) (end 131.2026 99.0953) (width 0.25) (layer B.Cu) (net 3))
 (segment (start 131.2026 99.0953) (end 130.3947 99.9032) (width 0.25) (layer B.Cu) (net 3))
 (segment (start 130.3947 99.9032) (end 130.3947 101.7381) (width 0.25) (layer B.Cu) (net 3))
 (segment (start 130.3947 101.7381) (end 135.9562 101.7381) (width 0.25) (layer B.Cu) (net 3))
 (segment (start 135.9562 101.7381) (end 139.4627 105.2446) (width 0.25) (layer B.Cu) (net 3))
 (segment (start 139.4627 105.2446) (end 179.3901 105.2446) (width 0.25) (layer B.Cu) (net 3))
 (segment (start 179.3901 105.2446) (end 181.4447 103.19) (width 0.25) (layer B.Cu) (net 3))
 (segment (start 182.57 103.19) (end 181.4447 103.19) (width 0.25) (layer B.Cu) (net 3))
 (segment (start 114.7 103.09) (end 115.8253 103.09) (width 0.25) (layer B.Cu) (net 3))
 (segment (start 131.57 97.92) (end 131.57 99.0953) (width 0.25) (layer B.Cu) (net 3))
 (segment (start 135.81 103.19) (end 134.6847 103.19) (width 0.25) (layer B.Cu) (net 7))
 (segment (start 131.57 103) (end 134.4947 103) (width 0.25) (layer B.Cu) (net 7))
 (segment (start 134.4947 103) (end 134.6847 103.19) (width 0.25) (layer B.Cu) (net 7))
 (segment (start 152.59 103.29) (end 153.7153 103.29) (width 0.25) (layer F.Cu) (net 12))
 (segment (start 165.41 100.97) (end 156.0353 100.97) (width 0.25) (layer F.Cu) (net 12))
 (segment (start 156.0353 100.97) (end 153.7153 103.29) (width 0.25) (layer F.Cu) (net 12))
 (segment (start 152.59 103.29) (end 151.4647 103.29) (width 0.25) (layer F.Cu) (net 12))
 (segment (start 118.75 103.19) (end 119.8753 103.19) (width 0.25) (layer F.Cu) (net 12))
 (segment (start 151.4647 103.29) (end 150.2032 104.5515) (width 0.25) (layer F.Cu) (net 12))
 (segment (start 150.2032 104.5515) (end 121.2368 104.5515) (width 0.25) (layer F.Cu) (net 12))
 (segment (start 121.2368 104.5515) (end 119.8753 103.19) (width 0.25) (layer F.Cu) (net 12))
 (segment (start 97.54 103) (end 98.6653 103) (width 0.25) (layer F.Cu) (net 12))
 (segment (start 118.75 103.19) (end 117.6247 103.19) (width 0.25) (layer F.Cu) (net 12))
 (segment (start 117.6247 103.19) (end 116.5551 104.2596) (width 0.25) (layer F.Cu) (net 12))
 (segment (start 116.5551 104.2596) (end 99.9249 104.2596) (width 0.25) (layer F.Cu) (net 12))
 (segment (start 99.9249 104.2596) (end 98.6653 103) (width 0.25) (layer F.Cu) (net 12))
 (segment (start 139.1447 101.6737) (end 140.211 102.74) (width 0.25) (layer F.Cu) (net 21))
 (segment (start 123.271 102.74) (end 124.5059 101.5051) (width 0.25) (layer F.Cu) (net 21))
 (segment (start 124.5059 101.5051) (end 128.1434 101.5051) (width 0.25) (layer F.Cu) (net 21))
 (segment (start 128.1434 101.5051) (end 128.312 101.6737) (width 0.25) (layer F.Cu) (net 21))
 (segment (start 128.312 101.6737) (end 139.1447 101.6737) (width 0.25) (layer F.Cu) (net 21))
 (segment (start 140.211 96.39) (end 140.6334 96.8124) (width 0.25) (layer F.Cu) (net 21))
 (segment (start 140.6334 96.8124) (end 140.6334 100.185) (width 0.25) (layer F.Cu) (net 21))
 (segment (start 140.6334 100.185) (end 139.1447 101.6737) (width 0.25) (layer F.Cu) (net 21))
 (segment (start 113.533 103.9676) (end 113.8833 104.3179) (width 0.25) (layer B.Cu) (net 21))
 (segment (start 113.8833 104.3179) (end 121.6931 104.3179) (width 0.25) (layer B.Cu) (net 21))
 (segment (start 121.6931 104.3179) (end 123.271 102.74) (width 0.25) (layer B.Cu) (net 21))
 (segment (start 113.533 103.9676) (end 113.533 102.6482) (width 0.25) (layer B.Cu) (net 21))
 (segment (start 113.533 102.6482) (end 118.9094 97.2718) (width 0.25) (layer B.Cu) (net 21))
 (segment (start 118.9094 97.2718) (end 122.3892 97.2718) (width 0.25) (layer B.Cu) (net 21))
 (segment (start 122.3892 97.2718) (end 123.271 96.39) (width 0.25) (layer B.Cu) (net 21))
 (segment (start 106.7678 102.3132) (end 108.4222 103.9676) (width 0.25) (layer B.Cu) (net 21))
 (segment (start 108.4222 103.9676) (end 113.533 103.9676) (width 0.25) (layer B.Cu) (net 21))
 (segment (start 106.7678 102.3132) (end 106.341 102.74) (width 0.25) (layer B.Cu) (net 21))
 (segment (start 106.341 96.39) (end 106.7678 96.8168) (width 0.25) (layer B.Cu) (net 21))
 (segment (start 106.7678 96.8168) (end 106.7678 102.3132) (width 0.25) (layer B.Cu) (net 21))
 (segment (start 89.411 96.39) (end 90.5925 97.5715) (width 0.25) (layer F.Cu) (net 21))
 (segment (start 90.5925 97.5715) (end 105.1595 97.5715) (width 0.25) (layer F.Cu) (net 21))
 (segment (start 105.1595 97.5715) (end 106.341 96.39) (width 0.25) (layer F.Cu) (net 21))
 (segment (start 89.411 96.39) (end 89.8274 96.8064) (width 0.25) (layer B.Cu) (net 21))
 (segment (start 89.8274 96.8064) (end 89.8274 102.3236) (width 0.25) (layer B.Cu) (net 21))
 (segment (start 89.8274 102.3236) (end 89.411 102.74) (width 0.25) (layer B.Cu) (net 21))
 (segment (start 165.6 97.34) (end 164.4247 97.34) (width 0.25) (layer B.Cu) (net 21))
 (segment (start 140.211 96.39) (end 142.0662 94.5348) (width 0.25) (layer B.Cu) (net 21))
 (segment (start 142.0662 94.5348) (end 161.6195 94.5348) (width 0.25) (layer B.Cu) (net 21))
 (segment (start 161.6195 94.5348) (end 164.4247 97.34) (width 0.25) (layer B.Cu) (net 21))
 (segment (start 174.071 96.39) (end 174.4673 96.7863) (width 0.25) (layer B.Cu) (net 18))
 (segment (start 174.4673 96.7863) (end 174.4673 102.3437) (width 0.25) (layer B.Cu) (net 18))
 (segment (start 174.4673 102.3437) (end 174.071 102.74) (width 0.25) (layer B.Cu) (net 18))
 (segment (start 166.7753 94.8) (end 167.1307 94.4446) (width 0.25) (layer B.Cu) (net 18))
 (segment (start 167.1307 94.4446) (end 172.1256 94.4446) (width 0.25) (layer B.Cu) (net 18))
 (segment (start 172.1256 94.4446) (end 174.071 96.39) (width 0.25) (layer B.Cu) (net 18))
 (segment (start 189.8269 97.5741) (end 191.011 96.39) (width 0.25) (layer F.Cu) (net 18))
 (segment (start 174.071 96.39) (end 175.2551 97.5741) (width 0.25) (layer F.Cu) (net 18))
 (segment (start 175.2551 97.5741) (end 189.8269 97.5741) (width 0.25) (layer F.Cu) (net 18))
 (segment (start 189.8269 97.5741) (end 191.4295 99.1767) (width 0.25) (layer F.Cu) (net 18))
 (segment (start 191.4295 99.1767) (end 191.4295 102.3215) (width 0.25) (layer F.Cu) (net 18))
 (segment (start 191.4295 102.3215) (end 191.011 102.74) (width 0.25) (layer F.Cu) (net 18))
 (segment (start 157.141 96.39) (end 157.5519 96.8009) (width 0.25) (layer B.Cu) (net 18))
 (segment (start 157.5519 96.8009) (end 157.5519 102.3291) (width 0.25) (layer B.Cu) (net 18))
 (segment (start 157.5519 102.3291) (end 157.141 102.74) (width 0.25) (layer B.Cu) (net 18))
 (segment (start 165.6 94.8) (end 166.7753 94.8) (width 0.25) (layer B.Cu) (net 18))
 (segment (start 165.6 94.8) (end 158.731 94.8) (width 0.25) (layer F.Cu) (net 18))
 (segment (start 158.731 94.8) (end 157.141 96.39) (width 0.25) (layer F.Cu) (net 18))
 (segment (start 139.5 99.605) (end 140.6355 98.4695) (width 0.25) (layer B.Cu) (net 16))
 (segment (start 140.6355 98.4695) (end 154.7731 98.4695) (width 0.25) (layer B.Cu) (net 16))
 (segment (start 154.7731 98.4695) (end 155.9086 99.605) (width 0.25) (layer B.Cu) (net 16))
 (segment (start 88.7 99.605) (end 89.846 98.459) (width 0.25) (layer F.Cu) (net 16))
 (segment (start 89.846 98.459) (end 108.2629 98.459) (width 0.25) (layer F.Cu) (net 16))
 (segment (start 108.2629 98.459) (end 110.4962 100.6923) (width 0.25) (layer F.Cu) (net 16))
 (segment (start 110.4962 100.6923) (end 123.197 100.6923) (width 0.25) (layer F.Cu) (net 16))
 (segment (start 123.197 100.6923) (end 125.4128 98.4765) (width 0.25) (layer F.Cu) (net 16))
 (segment (start 125.4128 98.4765) (end 129.5336 98.4765) (width 0.25) (layer F.Cu) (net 16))
 (segment (start 129.5336 98.4765) (end 130.2471 99.19) (width 0.25) (layer F.Cu) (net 16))
 (segment (start 130.2471 99.19) (end 139.085 99.19) (width 0.25) (layer F.Cu) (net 16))
 (segment (start 139.085 99.19) (end 139.5 99.605) (width 0.25) (layer F.Cu) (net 16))
 (segment (start 155.9086 99.605) (end 156.43 99.605) (width 0.25) (layer B.Cu) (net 16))
 (segment (start 155.9086 99.605) (end 155.9086 103.2287) (width 0.25) (layer B.Cu) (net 16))
 (segment (start 155.9086 103.2287) (end 156.6436 103.9637) (width 0.25) (layer B.Cu) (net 16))
 (segment (start 156.6436 103.9637) (end 163.781 103.9637) (width 0.25) (layer B.Cu) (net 16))
 (segment (start 163.781 103.9637) (end 164.2347 103.51) (width 0.25) (layer B.Cu) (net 16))
 (segment (start 165.41 103.51) (end 164.2347 103.51) (width 0.25) (layer B.Cu) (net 16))
 (segment (start 122.56 99.605) (end 124.21 97.955) (width 0.25) (layer F.Cu) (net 20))
 (segment (start 124.21 97.955) (end 128.6875 97.955) (width 0.25) (layer F.Cu) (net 20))
 (segment (start 128.6875 97.955) (end 129.947 96.6955) (width 0.25) (layer F.Cu) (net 20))
 (segment (start 129.947 96.6955) (end 137.1197 96.6955) (width 0.25) (layer F.Cu) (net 20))
 (segment (start 137.1197 96.6955) (end 138.6268 95.1884) (width 0.25) (layer F.Cu) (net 20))
 (segment (start 138.6268 95.1884) (end 140.9144 95.1884) (width 0.25) (layer F.Cu) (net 20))
 (segment (start 140.9144 95.1884) (end 145.291 99.565) (width 0.25) (layer F.Cu) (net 20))
 (segment (start 162.221 99.565) (end 173.32 99.565) (width 0.25) (layer B.Cu) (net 19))
 (segment (start 173.32 99.565) (end 173.36 99.605) (width 0.25) (layer B.Cu) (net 19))
 (segment (start 179.151 99.565) (end 190.26 99.565) (width 0.25) (layer F.Cu) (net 17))
 (segment (start 190.26 99.565) (end 190.3 99.605) (width 0.25) (layer F.Cu) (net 17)))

